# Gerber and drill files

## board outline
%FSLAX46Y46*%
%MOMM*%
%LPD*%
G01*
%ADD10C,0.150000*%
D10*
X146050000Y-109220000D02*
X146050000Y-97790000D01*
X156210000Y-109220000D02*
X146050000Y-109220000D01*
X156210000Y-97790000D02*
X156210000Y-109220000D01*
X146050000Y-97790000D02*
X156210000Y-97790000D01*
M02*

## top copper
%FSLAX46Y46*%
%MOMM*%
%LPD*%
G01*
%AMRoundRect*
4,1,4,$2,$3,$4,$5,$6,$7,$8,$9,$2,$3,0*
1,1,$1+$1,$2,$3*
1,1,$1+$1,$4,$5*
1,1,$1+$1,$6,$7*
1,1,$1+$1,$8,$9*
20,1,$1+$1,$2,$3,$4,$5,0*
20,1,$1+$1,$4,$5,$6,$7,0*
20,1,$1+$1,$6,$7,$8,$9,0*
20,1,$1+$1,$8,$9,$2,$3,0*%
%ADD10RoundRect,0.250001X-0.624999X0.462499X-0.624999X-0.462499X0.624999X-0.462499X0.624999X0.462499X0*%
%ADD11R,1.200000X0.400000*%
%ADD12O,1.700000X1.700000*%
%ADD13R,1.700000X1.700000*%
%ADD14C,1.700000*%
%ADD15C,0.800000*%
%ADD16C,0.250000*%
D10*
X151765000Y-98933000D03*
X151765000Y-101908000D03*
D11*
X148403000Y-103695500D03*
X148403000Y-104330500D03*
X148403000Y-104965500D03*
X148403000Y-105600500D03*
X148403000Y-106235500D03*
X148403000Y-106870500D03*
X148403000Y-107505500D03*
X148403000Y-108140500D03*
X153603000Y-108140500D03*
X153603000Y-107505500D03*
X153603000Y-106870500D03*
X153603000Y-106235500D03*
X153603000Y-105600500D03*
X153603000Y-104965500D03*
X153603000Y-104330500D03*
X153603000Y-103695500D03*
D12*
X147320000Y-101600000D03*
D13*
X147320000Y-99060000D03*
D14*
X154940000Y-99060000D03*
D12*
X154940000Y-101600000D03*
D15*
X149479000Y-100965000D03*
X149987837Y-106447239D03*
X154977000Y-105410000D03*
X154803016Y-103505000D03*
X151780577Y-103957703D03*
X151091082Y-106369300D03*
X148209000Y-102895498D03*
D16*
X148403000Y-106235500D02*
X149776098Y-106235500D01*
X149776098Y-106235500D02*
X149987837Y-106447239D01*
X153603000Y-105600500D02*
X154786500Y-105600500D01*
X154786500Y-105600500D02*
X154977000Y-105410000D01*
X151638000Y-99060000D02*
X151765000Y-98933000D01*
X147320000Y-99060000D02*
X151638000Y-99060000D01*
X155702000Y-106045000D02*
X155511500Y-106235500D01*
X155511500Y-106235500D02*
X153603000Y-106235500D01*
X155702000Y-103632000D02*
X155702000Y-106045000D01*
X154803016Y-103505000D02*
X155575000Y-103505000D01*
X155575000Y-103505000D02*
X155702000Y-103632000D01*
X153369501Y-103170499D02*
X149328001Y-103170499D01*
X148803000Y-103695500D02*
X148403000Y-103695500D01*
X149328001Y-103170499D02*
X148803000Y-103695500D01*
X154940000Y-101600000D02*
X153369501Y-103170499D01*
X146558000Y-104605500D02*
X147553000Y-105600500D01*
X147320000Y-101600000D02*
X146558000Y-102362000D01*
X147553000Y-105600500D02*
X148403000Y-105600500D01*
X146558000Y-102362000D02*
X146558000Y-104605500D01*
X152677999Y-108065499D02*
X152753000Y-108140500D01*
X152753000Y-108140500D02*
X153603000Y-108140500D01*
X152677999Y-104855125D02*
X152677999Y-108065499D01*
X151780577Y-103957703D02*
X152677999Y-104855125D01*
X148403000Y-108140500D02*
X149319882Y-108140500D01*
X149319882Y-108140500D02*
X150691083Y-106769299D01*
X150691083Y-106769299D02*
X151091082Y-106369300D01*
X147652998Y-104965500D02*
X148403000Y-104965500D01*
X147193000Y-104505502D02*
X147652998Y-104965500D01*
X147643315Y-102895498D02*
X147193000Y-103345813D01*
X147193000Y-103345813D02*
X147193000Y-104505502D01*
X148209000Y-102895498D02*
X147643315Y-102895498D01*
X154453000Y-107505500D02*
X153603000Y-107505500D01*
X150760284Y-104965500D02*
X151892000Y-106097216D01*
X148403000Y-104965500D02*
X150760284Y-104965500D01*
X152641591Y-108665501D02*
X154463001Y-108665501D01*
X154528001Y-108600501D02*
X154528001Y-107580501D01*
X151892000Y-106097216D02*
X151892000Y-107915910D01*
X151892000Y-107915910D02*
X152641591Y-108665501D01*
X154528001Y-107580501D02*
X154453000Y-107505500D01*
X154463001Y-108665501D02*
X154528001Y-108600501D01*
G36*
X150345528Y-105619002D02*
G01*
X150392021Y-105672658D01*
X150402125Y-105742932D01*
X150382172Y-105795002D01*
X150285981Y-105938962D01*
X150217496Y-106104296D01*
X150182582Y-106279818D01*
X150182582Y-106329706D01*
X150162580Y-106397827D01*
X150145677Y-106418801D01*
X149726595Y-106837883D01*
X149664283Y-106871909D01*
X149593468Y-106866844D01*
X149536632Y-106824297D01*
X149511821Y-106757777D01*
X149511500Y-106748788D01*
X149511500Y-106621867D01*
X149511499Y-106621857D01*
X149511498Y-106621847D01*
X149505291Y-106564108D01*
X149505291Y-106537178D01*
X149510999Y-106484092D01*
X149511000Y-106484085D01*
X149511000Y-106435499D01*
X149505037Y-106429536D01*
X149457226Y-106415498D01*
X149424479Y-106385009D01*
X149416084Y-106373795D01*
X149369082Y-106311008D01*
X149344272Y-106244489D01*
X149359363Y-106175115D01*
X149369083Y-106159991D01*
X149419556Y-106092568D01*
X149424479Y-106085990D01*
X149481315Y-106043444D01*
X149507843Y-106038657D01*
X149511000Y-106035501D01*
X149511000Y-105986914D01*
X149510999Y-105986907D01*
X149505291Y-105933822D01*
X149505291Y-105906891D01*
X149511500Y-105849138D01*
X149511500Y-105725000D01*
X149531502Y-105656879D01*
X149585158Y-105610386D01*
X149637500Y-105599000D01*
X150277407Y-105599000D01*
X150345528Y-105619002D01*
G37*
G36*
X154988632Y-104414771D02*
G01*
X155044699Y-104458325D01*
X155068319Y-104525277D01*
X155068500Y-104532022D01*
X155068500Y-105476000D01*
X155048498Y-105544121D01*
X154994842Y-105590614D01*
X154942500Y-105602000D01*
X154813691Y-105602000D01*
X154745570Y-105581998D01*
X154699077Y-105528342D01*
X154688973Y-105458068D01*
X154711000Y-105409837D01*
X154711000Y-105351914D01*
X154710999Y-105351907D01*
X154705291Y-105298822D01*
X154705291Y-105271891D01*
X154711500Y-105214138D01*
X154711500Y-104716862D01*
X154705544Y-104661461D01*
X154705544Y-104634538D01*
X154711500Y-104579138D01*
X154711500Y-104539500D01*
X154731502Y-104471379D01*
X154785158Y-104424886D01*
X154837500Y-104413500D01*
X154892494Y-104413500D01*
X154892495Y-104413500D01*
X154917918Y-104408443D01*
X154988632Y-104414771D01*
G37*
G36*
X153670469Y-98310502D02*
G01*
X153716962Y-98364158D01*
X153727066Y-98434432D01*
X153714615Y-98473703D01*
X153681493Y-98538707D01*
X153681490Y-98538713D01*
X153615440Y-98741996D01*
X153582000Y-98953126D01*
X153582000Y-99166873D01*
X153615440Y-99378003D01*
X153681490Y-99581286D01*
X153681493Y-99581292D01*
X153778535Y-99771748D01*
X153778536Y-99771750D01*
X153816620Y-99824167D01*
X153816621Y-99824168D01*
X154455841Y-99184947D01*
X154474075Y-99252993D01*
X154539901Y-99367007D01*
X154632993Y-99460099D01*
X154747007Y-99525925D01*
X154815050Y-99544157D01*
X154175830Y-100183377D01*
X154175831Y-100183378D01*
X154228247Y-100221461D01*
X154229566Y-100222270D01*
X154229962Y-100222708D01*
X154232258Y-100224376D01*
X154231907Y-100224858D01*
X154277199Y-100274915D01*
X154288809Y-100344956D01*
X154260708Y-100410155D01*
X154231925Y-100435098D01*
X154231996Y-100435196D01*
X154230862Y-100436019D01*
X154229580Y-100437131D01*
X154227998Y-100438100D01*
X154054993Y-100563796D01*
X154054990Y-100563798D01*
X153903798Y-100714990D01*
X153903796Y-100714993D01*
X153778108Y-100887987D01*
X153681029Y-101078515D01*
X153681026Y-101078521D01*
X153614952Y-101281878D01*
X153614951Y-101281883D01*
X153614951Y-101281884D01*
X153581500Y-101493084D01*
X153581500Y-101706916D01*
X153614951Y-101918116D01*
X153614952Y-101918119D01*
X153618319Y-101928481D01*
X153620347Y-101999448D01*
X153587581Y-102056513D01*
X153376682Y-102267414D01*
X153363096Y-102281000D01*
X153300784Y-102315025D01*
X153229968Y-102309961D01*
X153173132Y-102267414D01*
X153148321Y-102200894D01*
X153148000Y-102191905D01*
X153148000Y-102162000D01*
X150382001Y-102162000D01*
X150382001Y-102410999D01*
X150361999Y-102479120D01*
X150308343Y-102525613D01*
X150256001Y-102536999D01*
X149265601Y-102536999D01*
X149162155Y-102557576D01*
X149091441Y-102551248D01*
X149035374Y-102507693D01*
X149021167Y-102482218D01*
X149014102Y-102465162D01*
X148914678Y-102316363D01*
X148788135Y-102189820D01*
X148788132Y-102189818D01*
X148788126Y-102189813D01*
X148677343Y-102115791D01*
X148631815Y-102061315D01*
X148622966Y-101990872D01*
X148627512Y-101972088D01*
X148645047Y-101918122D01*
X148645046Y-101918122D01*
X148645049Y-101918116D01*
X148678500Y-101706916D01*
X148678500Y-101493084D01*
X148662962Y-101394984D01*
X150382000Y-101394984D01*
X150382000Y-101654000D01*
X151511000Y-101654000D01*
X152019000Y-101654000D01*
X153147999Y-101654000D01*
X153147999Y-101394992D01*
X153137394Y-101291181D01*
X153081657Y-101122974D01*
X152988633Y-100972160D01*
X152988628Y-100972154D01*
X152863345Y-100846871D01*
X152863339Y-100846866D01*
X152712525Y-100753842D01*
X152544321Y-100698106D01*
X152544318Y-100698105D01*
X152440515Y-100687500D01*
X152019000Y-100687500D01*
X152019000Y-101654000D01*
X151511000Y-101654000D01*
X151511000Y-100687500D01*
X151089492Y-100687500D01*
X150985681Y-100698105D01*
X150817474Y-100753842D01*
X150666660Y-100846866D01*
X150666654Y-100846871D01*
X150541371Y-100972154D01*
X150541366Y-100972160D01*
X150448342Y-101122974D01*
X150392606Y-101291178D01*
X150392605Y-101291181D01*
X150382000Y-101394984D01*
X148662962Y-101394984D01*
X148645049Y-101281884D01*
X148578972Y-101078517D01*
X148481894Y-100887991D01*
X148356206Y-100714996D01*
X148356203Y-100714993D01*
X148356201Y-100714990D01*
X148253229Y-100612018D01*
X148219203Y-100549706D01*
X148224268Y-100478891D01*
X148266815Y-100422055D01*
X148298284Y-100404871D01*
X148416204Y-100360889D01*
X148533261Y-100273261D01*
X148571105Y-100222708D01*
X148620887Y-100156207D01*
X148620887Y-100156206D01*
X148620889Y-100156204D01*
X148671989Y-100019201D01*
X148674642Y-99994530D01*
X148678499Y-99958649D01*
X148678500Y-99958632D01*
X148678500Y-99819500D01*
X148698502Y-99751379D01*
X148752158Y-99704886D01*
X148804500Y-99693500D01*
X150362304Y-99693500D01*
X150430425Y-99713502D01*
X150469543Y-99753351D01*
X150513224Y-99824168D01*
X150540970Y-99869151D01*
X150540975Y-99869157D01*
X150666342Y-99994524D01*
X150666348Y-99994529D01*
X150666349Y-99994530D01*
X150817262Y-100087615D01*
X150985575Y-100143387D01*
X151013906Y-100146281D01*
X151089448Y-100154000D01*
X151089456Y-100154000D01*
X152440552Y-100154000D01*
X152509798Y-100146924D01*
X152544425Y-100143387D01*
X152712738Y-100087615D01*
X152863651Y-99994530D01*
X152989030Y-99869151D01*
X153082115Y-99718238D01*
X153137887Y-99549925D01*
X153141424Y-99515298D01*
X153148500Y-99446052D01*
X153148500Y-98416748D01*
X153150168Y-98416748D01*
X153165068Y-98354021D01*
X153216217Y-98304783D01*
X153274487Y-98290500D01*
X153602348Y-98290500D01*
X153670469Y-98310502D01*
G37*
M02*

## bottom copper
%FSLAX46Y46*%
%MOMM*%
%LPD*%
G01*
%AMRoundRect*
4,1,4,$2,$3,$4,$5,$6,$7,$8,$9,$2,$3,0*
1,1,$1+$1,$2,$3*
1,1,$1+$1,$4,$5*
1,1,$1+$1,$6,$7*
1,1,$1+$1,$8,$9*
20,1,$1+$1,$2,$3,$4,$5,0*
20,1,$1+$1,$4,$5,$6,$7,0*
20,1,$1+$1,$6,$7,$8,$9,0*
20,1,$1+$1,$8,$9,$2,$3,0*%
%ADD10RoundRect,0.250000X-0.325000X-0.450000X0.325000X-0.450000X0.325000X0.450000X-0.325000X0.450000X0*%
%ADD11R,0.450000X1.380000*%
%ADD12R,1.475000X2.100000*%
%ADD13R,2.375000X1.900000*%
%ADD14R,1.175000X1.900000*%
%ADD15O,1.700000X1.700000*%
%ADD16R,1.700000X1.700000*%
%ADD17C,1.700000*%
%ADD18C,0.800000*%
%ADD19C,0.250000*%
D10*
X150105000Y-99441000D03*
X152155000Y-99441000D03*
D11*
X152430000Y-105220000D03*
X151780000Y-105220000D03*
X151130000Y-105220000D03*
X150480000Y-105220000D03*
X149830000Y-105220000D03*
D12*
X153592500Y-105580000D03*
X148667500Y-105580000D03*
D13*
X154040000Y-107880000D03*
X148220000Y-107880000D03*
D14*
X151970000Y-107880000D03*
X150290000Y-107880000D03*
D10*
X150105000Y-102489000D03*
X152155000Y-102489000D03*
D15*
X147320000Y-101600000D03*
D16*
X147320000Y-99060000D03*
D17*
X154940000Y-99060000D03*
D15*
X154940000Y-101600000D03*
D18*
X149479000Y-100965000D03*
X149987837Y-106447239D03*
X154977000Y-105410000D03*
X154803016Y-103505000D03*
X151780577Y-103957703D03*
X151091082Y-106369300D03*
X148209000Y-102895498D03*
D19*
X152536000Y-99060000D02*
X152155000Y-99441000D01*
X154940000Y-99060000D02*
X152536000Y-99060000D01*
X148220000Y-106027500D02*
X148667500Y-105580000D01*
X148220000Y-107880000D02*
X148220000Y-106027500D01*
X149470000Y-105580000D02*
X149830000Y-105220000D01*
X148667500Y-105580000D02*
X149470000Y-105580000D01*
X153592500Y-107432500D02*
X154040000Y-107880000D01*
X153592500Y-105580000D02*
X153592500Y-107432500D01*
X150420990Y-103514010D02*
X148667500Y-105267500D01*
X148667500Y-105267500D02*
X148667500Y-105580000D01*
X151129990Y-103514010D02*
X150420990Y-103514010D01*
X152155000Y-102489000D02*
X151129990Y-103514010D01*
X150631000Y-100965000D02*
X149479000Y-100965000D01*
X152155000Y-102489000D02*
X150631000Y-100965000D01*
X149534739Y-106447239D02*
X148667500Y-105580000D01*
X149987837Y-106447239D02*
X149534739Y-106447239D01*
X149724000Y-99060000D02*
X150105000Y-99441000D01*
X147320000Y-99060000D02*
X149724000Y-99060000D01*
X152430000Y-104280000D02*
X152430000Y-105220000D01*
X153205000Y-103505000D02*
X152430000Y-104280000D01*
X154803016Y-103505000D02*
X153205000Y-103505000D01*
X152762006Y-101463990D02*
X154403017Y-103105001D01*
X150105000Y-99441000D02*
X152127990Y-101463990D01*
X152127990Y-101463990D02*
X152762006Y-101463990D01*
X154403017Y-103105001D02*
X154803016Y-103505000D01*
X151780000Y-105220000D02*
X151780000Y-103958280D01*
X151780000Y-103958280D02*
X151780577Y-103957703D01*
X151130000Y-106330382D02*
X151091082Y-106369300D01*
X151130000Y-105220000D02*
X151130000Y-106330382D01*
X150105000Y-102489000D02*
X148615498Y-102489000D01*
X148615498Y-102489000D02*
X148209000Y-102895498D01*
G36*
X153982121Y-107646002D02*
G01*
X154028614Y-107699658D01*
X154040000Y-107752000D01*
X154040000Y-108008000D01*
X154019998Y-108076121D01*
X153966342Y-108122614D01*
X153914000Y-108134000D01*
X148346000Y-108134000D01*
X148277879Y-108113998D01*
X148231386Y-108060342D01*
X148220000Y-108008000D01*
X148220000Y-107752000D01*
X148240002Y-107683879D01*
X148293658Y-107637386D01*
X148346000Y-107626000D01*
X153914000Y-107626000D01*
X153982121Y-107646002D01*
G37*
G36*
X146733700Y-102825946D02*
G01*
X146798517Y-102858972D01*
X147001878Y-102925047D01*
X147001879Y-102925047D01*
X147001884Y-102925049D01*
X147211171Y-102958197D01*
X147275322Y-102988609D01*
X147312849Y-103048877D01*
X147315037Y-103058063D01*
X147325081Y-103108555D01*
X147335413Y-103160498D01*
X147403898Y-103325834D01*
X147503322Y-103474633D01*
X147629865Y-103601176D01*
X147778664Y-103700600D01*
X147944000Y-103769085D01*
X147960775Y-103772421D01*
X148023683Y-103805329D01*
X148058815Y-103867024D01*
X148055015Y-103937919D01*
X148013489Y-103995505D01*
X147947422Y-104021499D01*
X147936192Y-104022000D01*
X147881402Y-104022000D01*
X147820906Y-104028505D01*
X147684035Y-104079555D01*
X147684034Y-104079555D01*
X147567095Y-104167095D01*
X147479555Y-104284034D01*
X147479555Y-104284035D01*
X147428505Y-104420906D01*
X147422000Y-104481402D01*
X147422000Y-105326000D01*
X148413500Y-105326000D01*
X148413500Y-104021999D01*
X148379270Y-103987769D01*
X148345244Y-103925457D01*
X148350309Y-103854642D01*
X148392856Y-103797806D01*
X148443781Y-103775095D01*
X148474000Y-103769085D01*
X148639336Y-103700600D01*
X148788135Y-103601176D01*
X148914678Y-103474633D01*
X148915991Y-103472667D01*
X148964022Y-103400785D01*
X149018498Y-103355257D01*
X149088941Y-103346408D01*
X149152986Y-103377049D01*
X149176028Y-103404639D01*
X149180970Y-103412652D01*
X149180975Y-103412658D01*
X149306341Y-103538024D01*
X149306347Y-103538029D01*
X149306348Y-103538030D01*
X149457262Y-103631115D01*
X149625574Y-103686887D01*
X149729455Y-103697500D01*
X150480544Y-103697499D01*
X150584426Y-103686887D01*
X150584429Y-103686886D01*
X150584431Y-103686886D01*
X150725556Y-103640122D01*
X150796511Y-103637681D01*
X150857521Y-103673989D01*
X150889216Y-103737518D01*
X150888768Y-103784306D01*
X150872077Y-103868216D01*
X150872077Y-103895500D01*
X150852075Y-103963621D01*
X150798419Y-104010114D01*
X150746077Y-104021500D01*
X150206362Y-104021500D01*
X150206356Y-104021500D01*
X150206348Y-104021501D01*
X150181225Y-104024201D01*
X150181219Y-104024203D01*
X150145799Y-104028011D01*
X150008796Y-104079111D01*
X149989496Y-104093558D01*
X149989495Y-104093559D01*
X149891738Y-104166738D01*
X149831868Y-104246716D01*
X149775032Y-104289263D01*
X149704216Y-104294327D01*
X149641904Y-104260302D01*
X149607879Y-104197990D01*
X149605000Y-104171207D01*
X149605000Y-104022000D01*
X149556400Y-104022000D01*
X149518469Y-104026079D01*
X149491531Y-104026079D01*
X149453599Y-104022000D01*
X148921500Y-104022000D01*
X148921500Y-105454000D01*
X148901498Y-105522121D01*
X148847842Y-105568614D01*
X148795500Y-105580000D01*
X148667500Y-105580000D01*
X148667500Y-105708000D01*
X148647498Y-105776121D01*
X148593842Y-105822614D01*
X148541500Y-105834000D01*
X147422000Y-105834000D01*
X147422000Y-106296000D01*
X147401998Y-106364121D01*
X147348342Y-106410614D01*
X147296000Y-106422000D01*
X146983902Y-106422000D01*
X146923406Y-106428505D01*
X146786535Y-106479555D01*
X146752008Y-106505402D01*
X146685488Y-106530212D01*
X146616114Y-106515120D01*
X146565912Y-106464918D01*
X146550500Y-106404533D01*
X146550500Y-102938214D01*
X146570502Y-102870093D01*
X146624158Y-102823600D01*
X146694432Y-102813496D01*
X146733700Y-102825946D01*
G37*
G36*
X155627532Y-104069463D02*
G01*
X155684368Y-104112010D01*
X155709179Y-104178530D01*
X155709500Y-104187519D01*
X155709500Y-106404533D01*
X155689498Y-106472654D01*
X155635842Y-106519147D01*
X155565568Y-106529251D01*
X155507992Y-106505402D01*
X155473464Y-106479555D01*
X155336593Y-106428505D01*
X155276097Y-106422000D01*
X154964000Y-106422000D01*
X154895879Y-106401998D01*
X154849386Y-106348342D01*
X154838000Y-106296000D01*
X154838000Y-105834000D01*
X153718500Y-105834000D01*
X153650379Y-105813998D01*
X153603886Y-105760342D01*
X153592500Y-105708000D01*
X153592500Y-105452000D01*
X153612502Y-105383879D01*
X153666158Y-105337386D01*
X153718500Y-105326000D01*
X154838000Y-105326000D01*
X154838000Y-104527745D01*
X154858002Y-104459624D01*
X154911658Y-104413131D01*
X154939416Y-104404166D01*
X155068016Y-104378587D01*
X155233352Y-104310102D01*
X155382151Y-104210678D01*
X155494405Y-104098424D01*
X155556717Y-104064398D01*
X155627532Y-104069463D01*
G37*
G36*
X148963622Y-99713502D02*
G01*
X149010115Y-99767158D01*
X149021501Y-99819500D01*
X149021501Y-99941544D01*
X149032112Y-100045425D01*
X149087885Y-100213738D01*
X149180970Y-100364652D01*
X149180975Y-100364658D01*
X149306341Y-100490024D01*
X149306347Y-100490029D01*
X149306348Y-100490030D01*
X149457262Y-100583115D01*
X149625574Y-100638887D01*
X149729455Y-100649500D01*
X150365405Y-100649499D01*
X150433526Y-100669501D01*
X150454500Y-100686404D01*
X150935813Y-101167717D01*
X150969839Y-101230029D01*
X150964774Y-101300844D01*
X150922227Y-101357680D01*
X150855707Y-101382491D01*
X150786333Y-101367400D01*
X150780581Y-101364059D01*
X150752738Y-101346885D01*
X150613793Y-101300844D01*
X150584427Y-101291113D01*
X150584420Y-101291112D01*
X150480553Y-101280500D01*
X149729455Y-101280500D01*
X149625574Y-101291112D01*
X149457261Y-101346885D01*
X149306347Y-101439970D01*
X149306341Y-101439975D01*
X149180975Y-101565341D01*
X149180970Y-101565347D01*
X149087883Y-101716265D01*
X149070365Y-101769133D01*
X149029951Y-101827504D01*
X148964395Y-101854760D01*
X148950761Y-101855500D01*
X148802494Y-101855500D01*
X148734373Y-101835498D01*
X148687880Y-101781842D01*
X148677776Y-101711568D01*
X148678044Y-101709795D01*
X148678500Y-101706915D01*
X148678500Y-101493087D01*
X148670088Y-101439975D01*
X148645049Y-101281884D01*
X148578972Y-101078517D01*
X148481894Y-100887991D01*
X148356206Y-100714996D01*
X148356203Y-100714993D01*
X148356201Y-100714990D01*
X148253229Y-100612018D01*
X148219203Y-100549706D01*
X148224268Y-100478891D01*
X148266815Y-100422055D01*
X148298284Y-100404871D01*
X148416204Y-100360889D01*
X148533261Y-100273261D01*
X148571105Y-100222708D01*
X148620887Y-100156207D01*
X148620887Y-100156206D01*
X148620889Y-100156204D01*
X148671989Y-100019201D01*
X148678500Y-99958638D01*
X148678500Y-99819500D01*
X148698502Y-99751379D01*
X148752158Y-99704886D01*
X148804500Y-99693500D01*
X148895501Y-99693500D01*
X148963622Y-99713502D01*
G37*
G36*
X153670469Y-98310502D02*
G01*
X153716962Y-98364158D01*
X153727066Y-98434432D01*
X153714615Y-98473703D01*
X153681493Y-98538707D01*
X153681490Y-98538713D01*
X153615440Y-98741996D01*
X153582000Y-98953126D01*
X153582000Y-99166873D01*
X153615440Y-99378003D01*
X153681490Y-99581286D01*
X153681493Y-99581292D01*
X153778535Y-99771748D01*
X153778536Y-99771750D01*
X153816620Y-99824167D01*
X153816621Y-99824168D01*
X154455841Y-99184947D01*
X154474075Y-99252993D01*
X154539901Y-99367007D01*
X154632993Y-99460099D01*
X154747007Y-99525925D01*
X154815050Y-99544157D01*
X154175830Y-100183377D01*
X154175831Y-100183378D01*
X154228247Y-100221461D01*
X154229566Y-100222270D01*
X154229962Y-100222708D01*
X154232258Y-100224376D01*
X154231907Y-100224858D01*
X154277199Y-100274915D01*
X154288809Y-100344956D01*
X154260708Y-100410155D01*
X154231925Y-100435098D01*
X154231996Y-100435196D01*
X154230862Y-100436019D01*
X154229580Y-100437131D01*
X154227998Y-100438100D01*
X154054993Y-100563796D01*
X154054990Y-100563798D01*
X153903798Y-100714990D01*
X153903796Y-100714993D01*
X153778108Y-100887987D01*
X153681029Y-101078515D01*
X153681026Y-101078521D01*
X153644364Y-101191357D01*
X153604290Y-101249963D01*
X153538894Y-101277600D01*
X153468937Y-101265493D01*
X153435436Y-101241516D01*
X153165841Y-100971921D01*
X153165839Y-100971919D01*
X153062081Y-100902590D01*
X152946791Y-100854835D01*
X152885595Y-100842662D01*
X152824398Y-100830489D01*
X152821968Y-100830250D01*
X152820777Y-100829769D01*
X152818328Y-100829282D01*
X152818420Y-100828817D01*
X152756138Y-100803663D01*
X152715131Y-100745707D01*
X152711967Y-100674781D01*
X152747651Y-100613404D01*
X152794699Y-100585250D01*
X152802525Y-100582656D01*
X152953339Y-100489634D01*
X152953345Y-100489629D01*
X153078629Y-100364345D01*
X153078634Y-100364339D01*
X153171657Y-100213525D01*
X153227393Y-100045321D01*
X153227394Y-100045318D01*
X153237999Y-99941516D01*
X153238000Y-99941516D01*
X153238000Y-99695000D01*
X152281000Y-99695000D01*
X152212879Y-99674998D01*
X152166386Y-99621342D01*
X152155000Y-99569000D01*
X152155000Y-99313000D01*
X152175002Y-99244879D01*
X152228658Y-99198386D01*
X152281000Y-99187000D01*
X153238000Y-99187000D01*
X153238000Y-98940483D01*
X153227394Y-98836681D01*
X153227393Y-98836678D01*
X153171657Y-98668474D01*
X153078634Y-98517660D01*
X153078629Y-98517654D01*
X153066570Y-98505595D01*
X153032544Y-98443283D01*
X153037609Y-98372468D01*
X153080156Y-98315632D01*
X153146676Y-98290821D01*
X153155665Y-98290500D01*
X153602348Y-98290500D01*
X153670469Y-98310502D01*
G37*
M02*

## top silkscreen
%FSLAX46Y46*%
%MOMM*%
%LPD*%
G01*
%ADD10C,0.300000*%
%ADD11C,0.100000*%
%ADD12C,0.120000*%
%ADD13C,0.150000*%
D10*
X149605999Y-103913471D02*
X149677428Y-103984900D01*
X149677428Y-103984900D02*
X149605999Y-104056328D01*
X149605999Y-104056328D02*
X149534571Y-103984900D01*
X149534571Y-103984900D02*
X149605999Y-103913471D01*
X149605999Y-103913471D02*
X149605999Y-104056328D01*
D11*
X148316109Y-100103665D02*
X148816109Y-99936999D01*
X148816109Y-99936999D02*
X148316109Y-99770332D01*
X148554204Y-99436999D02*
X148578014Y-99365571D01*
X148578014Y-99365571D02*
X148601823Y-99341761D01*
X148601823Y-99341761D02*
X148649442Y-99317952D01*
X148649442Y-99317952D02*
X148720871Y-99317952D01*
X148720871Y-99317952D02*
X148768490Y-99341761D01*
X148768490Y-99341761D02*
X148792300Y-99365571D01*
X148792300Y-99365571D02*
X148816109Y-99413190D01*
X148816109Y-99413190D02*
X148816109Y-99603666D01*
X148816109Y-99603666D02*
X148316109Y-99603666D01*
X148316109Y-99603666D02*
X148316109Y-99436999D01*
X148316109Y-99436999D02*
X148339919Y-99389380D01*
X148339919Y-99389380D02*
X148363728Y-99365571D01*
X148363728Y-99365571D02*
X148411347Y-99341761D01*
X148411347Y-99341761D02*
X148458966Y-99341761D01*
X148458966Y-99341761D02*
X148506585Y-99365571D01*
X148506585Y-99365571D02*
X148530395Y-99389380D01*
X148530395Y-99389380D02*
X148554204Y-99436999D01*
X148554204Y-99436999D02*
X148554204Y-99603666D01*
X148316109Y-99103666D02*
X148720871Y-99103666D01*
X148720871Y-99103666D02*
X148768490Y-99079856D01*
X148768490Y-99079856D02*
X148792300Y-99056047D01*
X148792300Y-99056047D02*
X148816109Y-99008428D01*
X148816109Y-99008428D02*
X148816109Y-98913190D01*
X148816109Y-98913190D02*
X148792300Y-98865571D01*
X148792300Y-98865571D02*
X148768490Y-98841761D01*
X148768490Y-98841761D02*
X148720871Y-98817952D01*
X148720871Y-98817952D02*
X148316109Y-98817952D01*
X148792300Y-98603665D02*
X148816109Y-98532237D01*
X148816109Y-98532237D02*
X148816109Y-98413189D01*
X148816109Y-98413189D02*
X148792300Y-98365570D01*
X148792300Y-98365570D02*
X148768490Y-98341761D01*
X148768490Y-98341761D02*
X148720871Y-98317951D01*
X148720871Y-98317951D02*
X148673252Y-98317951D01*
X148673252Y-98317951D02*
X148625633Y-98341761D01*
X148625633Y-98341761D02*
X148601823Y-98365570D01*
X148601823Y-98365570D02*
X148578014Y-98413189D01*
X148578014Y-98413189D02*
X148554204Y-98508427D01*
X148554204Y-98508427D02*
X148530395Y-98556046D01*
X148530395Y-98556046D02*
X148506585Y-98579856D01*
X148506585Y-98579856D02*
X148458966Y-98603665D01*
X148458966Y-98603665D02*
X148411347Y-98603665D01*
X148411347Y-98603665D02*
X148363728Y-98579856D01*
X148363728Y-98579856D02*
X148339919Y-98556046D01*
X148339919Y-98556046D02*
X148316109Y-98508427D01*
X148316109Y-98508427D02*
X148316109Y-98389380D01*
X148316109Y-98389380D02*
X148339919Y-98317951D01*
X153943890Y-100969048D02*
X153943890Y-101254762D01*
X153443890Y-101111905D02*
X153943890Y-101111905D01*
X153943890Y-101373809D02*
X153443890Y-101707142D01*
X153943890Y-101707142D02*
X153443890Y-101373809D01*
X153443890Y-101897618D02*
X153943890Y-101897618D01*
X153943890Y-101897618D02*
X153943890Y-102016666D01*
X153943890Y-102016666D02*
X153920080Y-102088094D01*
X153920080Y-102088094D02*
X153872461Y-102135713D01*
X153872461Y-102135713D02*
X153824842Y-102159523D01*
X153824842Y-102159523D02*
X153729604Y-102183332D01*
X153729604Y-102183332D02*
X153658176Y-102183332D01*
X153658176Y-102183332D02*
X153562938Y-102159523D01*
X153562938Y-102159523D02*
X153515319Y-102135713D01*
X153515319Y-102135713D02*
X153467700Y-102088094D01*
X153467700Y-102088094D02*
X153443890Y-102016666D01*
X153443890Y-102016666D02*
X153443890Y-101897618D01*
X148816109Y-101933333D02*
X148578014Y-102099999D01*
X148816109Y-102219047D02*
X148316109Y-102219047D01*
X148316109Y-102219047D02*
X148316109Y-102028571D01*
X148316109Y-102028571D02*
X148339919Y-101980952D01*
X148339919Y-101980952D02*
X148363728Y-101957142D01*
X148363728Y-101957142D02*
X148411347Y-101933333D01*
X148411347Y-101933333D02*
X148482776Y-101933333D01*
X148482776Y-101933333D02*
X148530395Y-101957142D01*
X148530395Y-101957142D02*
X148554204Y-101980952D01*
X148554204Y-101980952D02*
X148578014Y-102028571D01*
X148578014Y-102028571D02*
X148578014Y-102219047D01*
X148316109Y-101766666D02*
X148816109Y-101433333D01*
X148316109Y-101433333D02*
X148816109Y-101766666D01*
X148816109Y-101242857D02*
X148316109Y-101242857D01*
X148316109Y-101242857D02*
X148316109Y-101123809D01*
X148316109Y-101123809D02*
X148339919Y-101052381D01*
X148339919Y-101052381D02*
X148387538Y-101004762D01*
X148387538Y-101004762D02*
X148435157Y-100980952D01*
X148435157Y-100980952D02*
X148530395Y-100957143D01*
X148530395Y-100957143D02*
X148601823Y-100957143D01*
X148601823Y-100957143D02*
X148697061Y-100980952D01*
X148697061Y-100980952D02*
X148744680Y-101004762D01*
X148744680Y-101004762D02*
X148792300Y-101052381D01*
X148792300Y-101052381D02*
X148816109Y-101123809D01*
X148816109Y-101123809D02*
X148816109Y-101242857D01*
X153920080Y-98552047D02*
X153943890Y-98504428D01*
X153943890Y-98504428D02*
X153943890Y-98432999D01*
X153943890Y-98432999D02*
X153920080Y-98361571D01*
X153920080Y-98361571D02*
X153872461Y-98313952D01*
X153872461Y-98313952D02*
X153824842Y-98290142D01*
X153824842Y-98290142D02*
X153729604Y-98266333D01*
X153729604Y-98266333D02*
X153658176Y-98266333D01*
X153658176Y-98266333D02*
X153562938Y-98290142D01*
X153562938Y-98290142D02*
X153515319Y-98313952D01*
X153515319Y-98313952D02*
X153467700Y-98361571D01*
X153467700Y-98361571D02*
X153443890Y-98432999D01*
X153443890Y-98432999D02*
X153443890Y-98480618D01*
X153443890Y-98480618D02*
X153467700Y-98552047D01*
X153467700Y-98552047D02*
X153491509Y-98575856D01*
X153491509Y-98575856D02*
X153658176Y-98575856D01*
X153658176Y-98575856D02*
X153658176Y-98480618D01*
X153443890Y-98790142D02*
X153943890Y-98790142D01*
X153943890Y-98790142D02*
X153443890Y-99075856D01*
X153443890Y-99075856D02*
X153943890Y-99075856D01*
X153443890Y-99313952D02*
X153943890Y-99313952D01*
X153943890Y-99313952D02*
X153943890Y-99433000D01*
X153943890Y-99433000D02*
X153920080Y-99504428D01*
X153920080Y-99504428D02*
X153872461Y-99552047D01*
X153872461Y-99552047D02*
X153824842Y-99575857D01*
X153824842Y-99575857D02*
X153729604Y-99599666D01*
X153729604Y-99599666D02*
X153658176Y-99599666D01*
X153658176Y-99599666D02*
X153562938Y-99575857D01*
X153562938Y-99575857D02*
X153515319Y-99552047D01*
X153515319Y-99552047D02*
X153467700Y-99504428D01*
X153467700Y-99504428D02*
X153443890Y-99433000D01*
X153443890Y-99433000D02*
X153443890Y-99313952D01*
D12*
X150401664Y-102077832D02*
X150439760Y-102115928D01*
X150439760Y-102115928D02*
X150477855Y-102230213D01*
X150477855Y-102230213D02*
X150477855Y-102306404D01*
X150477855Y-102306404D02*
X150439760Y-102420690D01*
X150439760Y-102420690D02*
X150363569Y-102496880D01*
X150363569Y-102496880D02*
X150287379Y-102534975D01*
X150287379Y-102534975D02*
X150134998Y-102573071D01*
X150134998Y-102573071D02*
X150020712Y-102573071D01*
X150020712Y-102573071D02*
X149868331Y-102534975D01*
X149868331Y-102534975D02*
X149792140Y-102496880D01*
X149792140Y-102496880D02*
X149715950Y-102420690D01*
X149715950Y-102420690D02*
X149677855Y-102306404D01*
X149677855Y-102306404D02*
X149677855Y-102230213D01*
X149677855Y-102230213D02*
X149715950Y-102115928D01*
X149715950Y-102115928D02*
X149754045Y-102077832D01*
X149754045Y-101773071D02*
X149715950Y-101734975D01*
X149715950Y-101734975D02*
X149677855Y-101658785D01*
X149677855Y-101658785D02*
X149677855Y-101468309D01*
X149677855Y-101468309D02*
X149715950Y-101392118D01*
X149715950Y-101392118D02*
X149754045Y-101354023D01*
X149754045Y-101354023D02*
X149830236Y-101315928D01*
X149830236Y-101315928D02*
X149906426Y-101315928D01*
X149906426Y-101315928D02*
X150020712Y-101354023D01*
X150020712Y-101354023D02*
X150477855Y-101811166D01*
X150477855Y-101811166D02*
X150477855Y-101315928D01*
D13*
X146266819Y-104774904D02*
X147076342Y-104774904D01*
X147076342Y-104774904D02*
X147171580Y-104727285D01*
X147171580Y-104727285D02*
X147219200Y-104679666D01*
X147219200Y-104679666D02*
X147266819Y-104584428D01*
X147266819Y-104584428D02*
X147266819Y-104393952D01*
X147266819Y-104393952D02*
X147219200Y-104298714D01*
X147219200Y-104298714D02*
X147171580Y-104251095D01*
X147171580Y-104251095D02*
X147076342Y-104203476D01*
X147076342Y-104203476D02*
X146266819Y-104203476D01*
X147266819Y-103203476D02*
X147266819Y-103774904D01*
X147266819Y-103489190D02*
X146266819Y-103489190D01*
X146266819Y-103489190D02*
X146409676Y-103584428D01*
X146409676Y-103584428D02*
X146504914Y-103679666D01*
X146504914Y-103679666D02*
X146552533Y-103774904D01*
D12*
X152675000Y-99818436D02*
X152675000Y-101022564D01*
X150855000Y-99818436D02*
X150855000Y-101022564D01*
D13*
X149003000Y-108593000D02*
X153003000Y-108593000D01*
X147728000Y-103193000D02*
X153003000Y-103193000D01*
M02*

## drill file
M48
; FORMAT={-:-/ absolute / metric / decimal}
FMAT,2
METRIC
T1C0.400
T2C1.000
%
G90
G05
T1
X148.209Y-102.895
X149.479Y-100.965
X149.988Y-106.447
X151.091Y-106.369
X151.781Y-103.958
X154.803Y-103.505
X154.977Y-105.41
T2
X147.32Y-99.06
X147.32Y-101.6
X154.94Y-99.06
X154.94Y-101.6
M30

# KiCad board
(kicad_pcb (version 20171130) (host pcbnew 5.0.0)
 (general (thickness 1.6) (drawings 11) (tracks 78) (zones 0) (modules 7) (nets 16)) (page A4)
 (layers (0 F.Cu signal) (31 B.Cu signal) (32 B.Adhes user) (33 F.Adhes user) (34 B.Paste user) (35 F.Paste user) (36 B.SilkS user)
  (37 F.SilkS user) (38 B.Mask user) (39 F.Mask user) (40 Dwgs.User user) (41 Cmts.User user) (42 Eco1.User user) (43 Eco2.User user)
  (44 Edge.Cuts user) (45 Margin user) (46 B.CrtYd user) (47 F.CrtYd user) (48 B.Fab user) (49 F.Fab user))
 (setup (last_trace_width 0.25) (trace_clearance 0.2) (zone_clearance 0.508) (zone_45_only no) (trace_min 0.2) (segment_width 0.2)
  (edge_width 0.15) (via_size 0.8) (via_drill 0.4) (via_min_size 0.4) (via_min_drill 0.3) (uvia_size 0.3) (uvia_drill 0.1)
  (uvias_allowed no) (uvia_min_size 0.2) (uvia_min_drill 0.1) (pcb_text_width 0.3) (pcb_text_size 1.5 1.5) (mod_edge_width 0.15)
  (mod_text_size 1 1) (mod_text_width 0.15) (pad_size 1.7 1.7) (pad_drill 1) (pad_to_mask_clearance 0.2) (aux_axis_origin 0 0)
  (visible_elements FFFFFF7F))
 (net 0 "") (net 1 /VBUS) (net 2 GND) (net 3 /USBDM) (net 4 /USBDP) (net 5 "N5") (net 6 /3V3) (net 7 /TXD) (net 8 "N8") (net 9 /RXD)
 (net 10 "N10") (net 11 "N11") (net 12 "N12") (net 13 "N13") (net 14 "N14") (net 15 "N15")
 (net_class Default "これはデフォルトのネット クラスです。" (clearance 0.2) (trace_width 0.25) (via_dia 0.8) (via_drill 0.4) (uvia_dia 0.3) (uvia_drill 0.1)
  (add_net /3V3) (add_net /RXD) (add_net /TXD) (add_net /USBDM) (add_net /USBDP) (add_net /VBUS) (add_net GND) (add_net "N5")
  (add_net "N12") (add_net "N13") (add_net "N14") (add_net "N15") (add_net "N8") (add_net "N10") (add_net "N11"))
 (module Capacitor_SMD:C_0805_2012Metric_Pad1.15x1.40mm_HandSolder (layer B.Cu) (at 151.13 99.441)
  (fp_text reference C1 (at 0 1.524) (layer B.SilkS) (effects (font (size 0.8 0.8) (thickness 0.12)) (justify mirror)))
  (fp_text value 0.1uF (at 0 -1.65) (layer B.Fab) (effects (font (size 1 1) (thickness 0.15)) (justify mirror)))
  (pad 1 smd roundrect (at -1.025 0) (size 1.15 1.4) (layers B.Cu B.Paste B.Mask) (roundrect_rratio 0.217391) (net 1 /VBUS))
  (pad 2 smd roundrect (at 1.025 0) (size 1.15 1.4) (layers B.Cu B.Paste B.Mask) (roundrect_rratio 0.217391) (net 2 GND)))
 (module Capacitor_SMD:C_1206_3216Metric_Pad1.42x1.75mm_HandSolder (layer F.Cu) (at 151.765 100.4205 270)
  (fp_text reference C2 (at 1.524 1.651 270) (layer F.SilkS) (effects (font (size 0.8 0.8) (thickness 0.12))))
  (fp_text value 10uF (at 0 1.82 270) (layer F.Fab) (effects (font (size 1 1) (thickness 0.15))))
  (fp_line (start -0.602064 -0.91) (end 0.602064 -0.91) (layer F.SilkS) (width 0.12))
  (fp_line (start -0.602064 0.91) (end 0.602064 0.91) (layer F.SilkS) (width 0.12))
  (pad 1 smd roundrect (at -1.4875 0 270) (size 1.425 1.75) (layers F.Cu F.Paste F.Mask) (roundrect_rratio 0.175439) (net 1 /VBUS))
  (pad 2 smd roundrect (at 1.4875 0 270) (size 1.425 1.75) (layers F.Cu F.Paste F.Mask) (roundrect_rratio 0.175439) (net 2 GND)))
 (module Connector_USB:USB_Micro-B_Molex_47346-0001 (layer B.Cu) (at 151.13 106.68 180)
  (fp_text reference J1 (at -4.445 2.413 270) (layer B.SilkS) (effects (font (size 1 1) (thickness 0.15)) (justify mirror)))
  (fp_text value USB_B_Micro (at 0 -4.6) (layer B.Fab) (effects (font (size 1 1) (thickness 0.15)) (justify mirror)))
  (pad 1 smd rect (at -1.3 1.46 180) (size 0.45 1.38) (layers B.Cu B.Paste B.Mask) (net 1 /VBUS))
  (pad 2 smd rect (at -0.65 1.46 180) (size 0.45 1.38) (layers B.Cu B.Paste B.Mask) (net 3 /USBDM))
  (pad 3 smd rect (at 0 1.46 180) (size 0.45 1.38) (layers B.Cu B.Paste B.Mask) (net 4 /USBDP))
  (pad 4 smd rect (at 0.65 1.46 180) (size 0.45 1.38) (layers B.Cu B.Paste B.Mask) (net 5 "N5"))
  (pad 5 smd rect (at 1.3 1.46 180) (size 0.45 1.38) (layers B.Cu B.Paste B.Mask) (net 2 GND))
  (pad 6 smd rect (at -2.4625 1.1 180) (size 1.475 2.1) (layers B.Cu B.Paste B.Mask) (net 2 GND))
  (pad 6 smd rect (at 2.4625 1.1 180) (size 1.475 2.1) (layers B.Cu B.Paste B.Mask) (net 2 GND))
  (pad 6 smd rect (at -2.91 -1.2 180) (size 2.375 1.9) (layers B.Cu B.Paste B.Mask) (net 2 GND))
  (pad 6 smd rect (at 2.91 -1.2 180) (size 2.375 1.9) (layers B.Cu B.Paste B.Mask) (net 2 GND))
  (pad 6 smd rect (at -0.84 -1.2 180) (size 1.175 1.9) (layers B.Cu B.Paste B.Mask) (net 2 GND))
  (pad 6 smd rect (at 0.84 -1.2 180) (size 1.175 1.9) (layers B.Cu B.Paste B.Mask) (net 2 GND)))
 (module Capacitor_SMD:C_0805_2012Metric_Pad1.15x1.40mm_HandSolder (layer B.Cu) (at 151.13 102.489)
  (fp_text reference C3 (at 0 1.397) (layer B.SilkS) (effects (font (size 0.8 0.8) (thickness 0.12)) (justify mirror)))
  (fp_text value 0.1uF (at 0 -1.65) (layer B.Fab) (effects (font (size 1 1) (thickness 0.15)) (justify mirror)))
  (pad 1 smd roundrect (at -1.025 0) (size 1.15 1.4) (layers B.Cu B.Paste B.Mask) (roundrect_rratio 0.217391) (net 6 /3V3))
  (pad 2 smd roundrect (at 1.025 0) (size 1.15 1.4) (layers B.Cu B.Paste B.Mask) (roundrect_rratio 0.217391) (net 2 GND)))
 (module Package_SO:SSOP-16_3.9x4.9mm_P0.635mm (layer F.Cu) (at 151.003 105.918)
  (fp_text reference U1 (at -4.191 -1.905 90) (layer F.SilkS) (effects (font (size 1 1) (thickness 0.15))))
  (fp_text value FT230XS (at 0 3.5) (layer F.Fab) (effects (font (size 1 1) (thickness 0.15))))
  (fp_line (start -2 2.675) (end 2 2.675) (layer F.SilkS) (width 0.15))
  (fp_line (start -3.275 -2.725) (end 2 -2.725) (layer F.SilkS) (width 0.15))
  (pad 1 smd rect (at -2.6 -2.2225) (size 1.2 0.4) (layers F.Cu F.Paste F.Mask) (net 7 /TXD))
  (pad 2 smd rect (at -2.6 -1.5875) (size 1.2 0.4) (layers F.Cu F.Paste F.Mask) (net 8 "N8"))
  (pad 3 smd rect (at -2.6 -0.9525) (size 1.2 0.4) (layers F.Cu F.Paste F.Mask) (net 6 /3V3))
  (pad 4 smd rect (at -2.6 -0.3175) (size 1.2 0.4) (layers F.Cu F.Paste F.Mask) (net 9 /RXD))
  (pad 5 smd rect (at -2.6 0.3175) (size 1.2 0.4) (layers F.Cu F.Paste F.Mask) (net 2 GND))
  (pad 6 smd rect (at -2.6 0.9525) (size 1.2 0.4) (layers F.Cu F.Paste F.Mask) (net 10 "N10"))
  (pad 7 smd rect (at -2.6 1.5875) (size 1.2 0.4) (layers F.Cu F.Paste F.Mask) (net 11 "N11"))
  (pad 8 smd rect (at -2.6 2.2225) (size 1.2 0.4) (layers F.Cu F.Paste F.Mask) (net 4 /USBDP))
  (pad 9 smd rect (at 2.6 2.2225) (size 1.2 0.4) (layers F.Cu F.Paste F.Mask) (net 3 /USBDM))
  (pad 10 smd rect (at 2.6 1.5875) (size 1.2 0.4) (layers F.Cu F.Paste F.Mask) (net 6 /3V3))
  (pad 11 smd rect (at 2.6 0.9525) (size 1.2 0.4) (layers F.Cu F.Paste F.Mask) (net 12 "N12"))
  (pad 12 smd rect (at 2.6 0.3175) (size 1.2 0.4) (layers F.Cu F.Paste F.Mask) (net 1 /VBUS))
  (pad 13 smd rect (at 2.6 -0.3175) (size 1.2 0.4) (layers F.Cu F.Paste F.Mask) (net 2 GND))
  (pad 14 smd rect (at 2.6 -0.9525) (size 1.2 0.4) (layers F.Cu F.Paste F.Mask) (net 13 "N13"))
  (pad 15 smd rect (at 2.6 -1.5875) (size 1.2 0.4) (layers F.Cu F.Paste F.Mask) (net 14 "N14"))
  (pad 16 smd rect (at 2.6 -2.2225) (size 1.2 0.4) (layers F.Cu F.Paste F.Mask) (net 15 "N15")))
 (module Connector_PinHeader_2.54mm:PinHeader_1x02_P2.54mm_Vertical (layer B.Cu) (at 147.32 99.06 180)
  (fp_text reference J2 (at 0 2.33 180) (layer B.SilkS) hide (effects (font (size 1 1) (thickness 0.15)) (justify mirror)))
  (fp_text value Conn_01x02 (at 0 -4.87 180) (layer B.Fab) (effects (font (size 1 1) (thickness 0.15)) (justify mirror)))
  (pad 2 thru_hole oval (at 0 -2.54 180) (size 1.7 1.7) (drill 1) (layers *.Cu *.Mask) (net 9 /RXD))
  (pad 1 thru_hole rect (at 0 0 180) (size 1.7 1.7) (drill 1) (layers *.Cu *.Mask) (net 1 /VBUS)))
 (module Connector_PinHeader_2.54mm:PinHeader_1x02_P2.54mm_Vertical (layer B.Cu) (at 154.94 99.06 180)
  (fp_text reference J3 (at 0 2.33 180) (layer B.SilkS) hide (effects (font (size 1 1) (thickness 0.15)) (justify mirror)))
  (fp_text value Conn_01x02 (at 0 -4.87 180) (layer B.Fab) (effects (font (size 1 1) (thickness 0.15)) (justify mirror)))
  (pad 1 thru_hole circle (at 0 0 180) (size 1.7 1.7) (drill 1) (layers *.Cu *.Mask) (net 2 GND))
  (pad 2 thru_hole oval (at 0 -2.54 180) (size 1.7 1.7) (drill 1) (layers *.Cu *.Mask) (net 7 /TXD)))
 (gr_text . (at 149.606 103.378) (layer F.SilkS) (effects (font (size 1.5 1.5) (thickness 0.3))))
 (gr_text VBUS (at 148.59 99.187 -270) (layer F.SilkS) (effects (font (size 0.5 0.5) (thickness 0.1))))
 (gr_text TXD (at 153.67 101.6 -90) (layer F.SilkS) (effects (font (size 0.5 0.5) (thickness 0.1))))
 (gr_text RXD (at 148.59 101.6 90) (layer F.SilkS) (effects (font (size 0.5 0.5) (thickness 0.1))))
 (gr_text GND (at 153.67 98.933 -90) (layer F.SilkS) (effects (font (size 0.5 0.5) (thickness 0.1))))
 (gr_line (start 146.05 109.22) (end 146.05 97.79) (layer Edge.Cuts) (width 0.15))
 (gr_line (start 156.21 109.22) (end 146.05 109.22) (layer Edge.Cuts) (width 0.15))
 (gr_line (start 156.21 97.79) (end 156.21 109.22) (layer Edge.Cuts) (width 0.15))
 (gr_line (start 146.05 97.79) (end 156.21 97.79) (layer Edge.Cuts) (width 0.15))
 (segment (start 152.536 99.06) (end 152.155 99.441) (width 0.25) (layer B.Cu) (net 2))
 (segment (start 154.94 99.06) (end 152.536 99.06) (width 0.25) (layer B.Cu) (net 2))
 (segment (start 148.22 106.0275) (end 148.6675 105.58) (width 0.25) (layer B.Cu) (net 2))
 (segment (start 148.22 107.88) (end 148.22 106.0275) (width 0.25) (layer B.Cu) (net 2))
 (segment (start 149.47 105.58) (end 149.83 105.22) (width 0.25) (layer B.Cu) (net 2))
 (segment (start 148.6675 105.58) (end 149.47 105.58) (width 0.25) (layer B.Cu) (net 2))
 (segment (start 153.5925 107.4325) (end 154.04 107.88) (width 0.25) (layer B.Cu) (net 2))
 (segment (start 153.5925 105.58) (end 153.5925 107.4325) (width 0.25) (layer B.Cu) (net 2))
 (segment (start 150.42099 103.51401) (end 148.6675 105.2675) (width 0.25) (layer B.Cu) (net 2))
 (segment (start 148.6675 105.2675) (end 148.6675 105.58) (width 0.25) (layer B.Cu) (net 2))
 (segment (start 151.12999 103.51401) (end 150.42099 103.51401) (width 0.25) (layer B.Cu) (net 2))
 (segment (start 152.155 102.489) (end 151.12999 103.51401) (width 0.25) (layer B.Cu) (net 2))
 (via (at 149.479 100.965) (size 0.8) (drill 0.4) (layers F.Cu B.Cu) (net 2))
 (segment (start 150.631 100.965) (end 149.479 100.965) (width 0.25) (layer B.Cu) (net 2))
 (segment (start 152.155 102.489) (end 150.631 100.965) (width 0.25) (layer B.Cu) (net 2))
 (via (at 149.987837 106.447239) (size 0.8) (drill 0.4) (layers F.Cu B.Cu) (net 2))
 (segment (start 148.403 106.2355) (end 149.776098 106.2355) (width 0.25) (layer F.Cu) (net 2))
 (segment (start 149.776098 106.2355) (end 149.987837 106.447239) (width 0.25) (layer F.Cu) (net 2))
 (segment (start 149.534739 106.447239) (end 148.6675 105.58) (width 0.25) (layer B.Cu) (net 2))
 (segment (start 149.987837 106.447239) (end 149.534739 106.447239) (width 0.25) (layer B.Cu) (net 2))
 (via (at 154.977 105.41) (size 0.8) (drill 0.4) (layers F.Cu B.Cu) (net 2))
 (segment (start 153.603 105.6005) (end 154.7865 105.6005) (width 0.25) (layer F.Cu) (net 2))
 (segment (start 154.7865 105.6005) (end 154.977 105.41) (width 0.25) (layer F.Cu) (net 2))
 (segment (start 151.638 99.06) (end 151.765 98.933) (width 0.25) (layer F.Cu) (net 1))
 (segment (start 147.32 99.06) (end 151.638 99.06) (width 0.25) (layer F.Cu) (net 1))
 (segment (start 149.724 99.06) (end 150.105 99.441) (width 0.25) (layer B.Cu) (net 1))
 (segment (start 147.32 99.06) (end 149.724 99.06) (width 0.25) (layer B.Cu) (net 1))
 (via (at 154.803016 103.505) (size 0.8) (drill 0.4) (layers F.Cu B.Cu) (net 1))
 (segment (start 152.43 104.28) (end 152.43 105.22) (width 0.25) (layer B.Cu) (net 1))
 (segment (start 153.205 103.505) (end 152.43 104.28) (width 0.25) (layer B.Cu) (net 1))
 (segment (start 154.803016 103.505) (end 153.205 103.505) (width 0.25) (layer B.Cu) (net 1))
 (segment (start 152.762006 101.46399) (end 154.403017 103.105001) (width 0.25) (layer B.Cu) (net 1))
 (segment (start 150.105 99.441) (end 152.12799 101.46399) (width 0.25) (layer B.Cu) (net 1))
 (segment (start 152.12799 101.46399) (end 152.762006 101.46399) (width 0.25) (layer B.Cu) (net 1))
 (segment (start 154.403017 103.105001) (end 154.803016 103.505) (width 0.25) (layer B.Cu) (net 1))
 (segment (start 155.702 106.045) (end 155.5115 106.2355) (width 0.25) (layer F.Cu) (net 1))
 (segment (start 155.5115 106.2355) (end 153.603 106.2355) (width 0.25) (layer F.Cu) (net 1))
 (segment (start 155.702 103.632) (end 155.702 106.045) (width 0.25) (layer F.Cu) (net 1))
 (segment (start 154.803016 103.505) (end 155.575 103.505) (width 0.25) (layer F.Cu) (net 1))
 (segment (start 155.575 103.505) (end 155.702 103.632) (width 0.25) (layer F.Cu) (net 1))
 (segment (start 153.369501 103.170499) (end 149.328001 103.170499) (width 0.25) (layer F.Cu) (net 7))
 (segment (start 148.803 103.6955) (end 148.403 103.6955) (width 0.25) (layer F.Cu) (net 7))
 (segment (start 149.328001 103.170499) (end 148.803 103.6955) (width 0.25) (layer F.Cu) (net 7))
 (segment (start 154.94 101.6) (end 153.369501 103.170499) (width 0.25) (layer F.Cu) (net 7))
 (segment (start 146.558 104.6055) (end 147.553 105.6005) (width 0.25) (layer F.Cu) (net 9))
 (segment (start 147.32 101.6) (end 146.558 102.362) (width 0.25) (layer F.Cu) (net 9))
 (segment (start 147.553 105.6005) (end 148.403 105.6005) (width 0.25) (layer F.Cu) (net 9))
 (segment (start 146.558 102.362) (end 146.558 104.6055) (width 0.25) (layer F.Cu) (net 9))
 (via (at 151.780577 103.957703) (size 0.8) (drill 0.4) (layers F.Cu B.Cu) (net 3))
 (segment (start 151.78 105.22) (end 151.78 103.95828) (width 0.25) (layer B.Cu) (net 3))
 (segment (start 151.78 103.95828) (end 151.780577 103.957703) (width 0.25) (layer B.Cu) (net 3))
 (segment (start 152.677999 108.065499) (end 152.753 108.1405) (width 0.25) (layer F.Cu) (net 3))
 (segment (start 152.753 108.1405) (end 153.603 108.1405) (width 0.25) (layer F.Cu) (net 3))
 (segment (start 152.677999 104.855125) (end 152.677999 108.065499) (width 0.25) (layer F.Cu) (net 3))
 (segment (start 151.780577 103.957703) (end 152.677999 104.855125) (width 0.25) (layer F.Cu) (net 3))
 (via (at 151.091082 106.3693) (size 0.8) (drill 0.4) (layers F.Cu B.Cu) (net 4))
 (segment (start 148.403 108.1405) (end 149.319882 108.1405) (width 0.25) (layer F.Cu) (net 4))
 (segment (start 149.319882 108.1405) (end 150.691083 106.769299) (width 0.25) (layer F.Cu) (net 4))
 (segment (start 150.691083 106.769299) (end 151.091082 106.3693) (width 0.25) (layer F.Cu) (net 4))
 (segment (start 151.13 106.330382) (end 151.091082 106.3693) (width 0.25) (layer B.Cu) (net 4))
 (segment (start 151.13 105.22) (end 151.13 106.330382) (width 0.25) (layer B.Cu) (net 4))
 (via (at 148.209 102.895498) (size 0.8) (drill 0.4) (layers F.Cu B.Cu) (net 6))
 (segment (start 150.105 102.489) (end 148.615498 102.489) (width 0.25) (layer B.Cu) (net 6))
 (segment (start 148.615498 102.489) (end 148.209 102.895498) (width 0.25) (layer B.Cu) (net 6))
 (segment (start 147.652998 104.9655) (end 148.403 104.9655) (width 0.25) (layer F.Cu) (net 6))
 (segment (start 147.193 104.505502) (end 147.652998 104.9655) (width 0.25) (layer F.Cu) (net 6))
 (segment (start 147.643315 102.895498) (end 147.193 103.345813) (width 0.25) (layer F.Cu) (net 6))
 (segment (start 147.193 103.345813) (end 147.193 104.505502) (width 0.25) (layer F.Cu) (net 6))
 (segment (start 148.209 102.895498) (end 147.643315 102.895498) (width 0.25) (layer F.Cu) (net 6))
 (segment (start 154.453 107.5055) (end 153.603 107.5055) (width 0.25) (layer F.Cu) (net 6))
 (segment (start 150.760284 104.9655) (end 151.892 106.097216) (width 0.25) (layer F.Cu) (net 6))
 (segment (start 148.403 104.9655) (end 150.760284 104.9655) (width 0.25) (layer F.Cu) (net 6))
 (segment (start 152.641591 108.665501) (end 154.463001 108.665501) (width 0.25) (layer F.Cu) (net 6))
 (segment (start 154.528001 108.600501) (end 154.528001 107.580501) (width 0.25) (layer F.Cu) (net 6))
 (segment (start 151.892 106.097216) (end 151.892 107.91591) (width 0.25) (layer F.Cu) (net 6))
 (segment (start 151.892 107.91591) (end 152.641591 108.665501) (width 0.25) (layer F.Cu) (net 6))
 (segment (start 154.528001 107.580501) (end 154.453 107.5055) (width 0.25) (layer F.Cu) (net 6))
 (segment (start 154.463001 108.665501) (end 154.528001 108.600501) (width 0.25) (layer F.Cu) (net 6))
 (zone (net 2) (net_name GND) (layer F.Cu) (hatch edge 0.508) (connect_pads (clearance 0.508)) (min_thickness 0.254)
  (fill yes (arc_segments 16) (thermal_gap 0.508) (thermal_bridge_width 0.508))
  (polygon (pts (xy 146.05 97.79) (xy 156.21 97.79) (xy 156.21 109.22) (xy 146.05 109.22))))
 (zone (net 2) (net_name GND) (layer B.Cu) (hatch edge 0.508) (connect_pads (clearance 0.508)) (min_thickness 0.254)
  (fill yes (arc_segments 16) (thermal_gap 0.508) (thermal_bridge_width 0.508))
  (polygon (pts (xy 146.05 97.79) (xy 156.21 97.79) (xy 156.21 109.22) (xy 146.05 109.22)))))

